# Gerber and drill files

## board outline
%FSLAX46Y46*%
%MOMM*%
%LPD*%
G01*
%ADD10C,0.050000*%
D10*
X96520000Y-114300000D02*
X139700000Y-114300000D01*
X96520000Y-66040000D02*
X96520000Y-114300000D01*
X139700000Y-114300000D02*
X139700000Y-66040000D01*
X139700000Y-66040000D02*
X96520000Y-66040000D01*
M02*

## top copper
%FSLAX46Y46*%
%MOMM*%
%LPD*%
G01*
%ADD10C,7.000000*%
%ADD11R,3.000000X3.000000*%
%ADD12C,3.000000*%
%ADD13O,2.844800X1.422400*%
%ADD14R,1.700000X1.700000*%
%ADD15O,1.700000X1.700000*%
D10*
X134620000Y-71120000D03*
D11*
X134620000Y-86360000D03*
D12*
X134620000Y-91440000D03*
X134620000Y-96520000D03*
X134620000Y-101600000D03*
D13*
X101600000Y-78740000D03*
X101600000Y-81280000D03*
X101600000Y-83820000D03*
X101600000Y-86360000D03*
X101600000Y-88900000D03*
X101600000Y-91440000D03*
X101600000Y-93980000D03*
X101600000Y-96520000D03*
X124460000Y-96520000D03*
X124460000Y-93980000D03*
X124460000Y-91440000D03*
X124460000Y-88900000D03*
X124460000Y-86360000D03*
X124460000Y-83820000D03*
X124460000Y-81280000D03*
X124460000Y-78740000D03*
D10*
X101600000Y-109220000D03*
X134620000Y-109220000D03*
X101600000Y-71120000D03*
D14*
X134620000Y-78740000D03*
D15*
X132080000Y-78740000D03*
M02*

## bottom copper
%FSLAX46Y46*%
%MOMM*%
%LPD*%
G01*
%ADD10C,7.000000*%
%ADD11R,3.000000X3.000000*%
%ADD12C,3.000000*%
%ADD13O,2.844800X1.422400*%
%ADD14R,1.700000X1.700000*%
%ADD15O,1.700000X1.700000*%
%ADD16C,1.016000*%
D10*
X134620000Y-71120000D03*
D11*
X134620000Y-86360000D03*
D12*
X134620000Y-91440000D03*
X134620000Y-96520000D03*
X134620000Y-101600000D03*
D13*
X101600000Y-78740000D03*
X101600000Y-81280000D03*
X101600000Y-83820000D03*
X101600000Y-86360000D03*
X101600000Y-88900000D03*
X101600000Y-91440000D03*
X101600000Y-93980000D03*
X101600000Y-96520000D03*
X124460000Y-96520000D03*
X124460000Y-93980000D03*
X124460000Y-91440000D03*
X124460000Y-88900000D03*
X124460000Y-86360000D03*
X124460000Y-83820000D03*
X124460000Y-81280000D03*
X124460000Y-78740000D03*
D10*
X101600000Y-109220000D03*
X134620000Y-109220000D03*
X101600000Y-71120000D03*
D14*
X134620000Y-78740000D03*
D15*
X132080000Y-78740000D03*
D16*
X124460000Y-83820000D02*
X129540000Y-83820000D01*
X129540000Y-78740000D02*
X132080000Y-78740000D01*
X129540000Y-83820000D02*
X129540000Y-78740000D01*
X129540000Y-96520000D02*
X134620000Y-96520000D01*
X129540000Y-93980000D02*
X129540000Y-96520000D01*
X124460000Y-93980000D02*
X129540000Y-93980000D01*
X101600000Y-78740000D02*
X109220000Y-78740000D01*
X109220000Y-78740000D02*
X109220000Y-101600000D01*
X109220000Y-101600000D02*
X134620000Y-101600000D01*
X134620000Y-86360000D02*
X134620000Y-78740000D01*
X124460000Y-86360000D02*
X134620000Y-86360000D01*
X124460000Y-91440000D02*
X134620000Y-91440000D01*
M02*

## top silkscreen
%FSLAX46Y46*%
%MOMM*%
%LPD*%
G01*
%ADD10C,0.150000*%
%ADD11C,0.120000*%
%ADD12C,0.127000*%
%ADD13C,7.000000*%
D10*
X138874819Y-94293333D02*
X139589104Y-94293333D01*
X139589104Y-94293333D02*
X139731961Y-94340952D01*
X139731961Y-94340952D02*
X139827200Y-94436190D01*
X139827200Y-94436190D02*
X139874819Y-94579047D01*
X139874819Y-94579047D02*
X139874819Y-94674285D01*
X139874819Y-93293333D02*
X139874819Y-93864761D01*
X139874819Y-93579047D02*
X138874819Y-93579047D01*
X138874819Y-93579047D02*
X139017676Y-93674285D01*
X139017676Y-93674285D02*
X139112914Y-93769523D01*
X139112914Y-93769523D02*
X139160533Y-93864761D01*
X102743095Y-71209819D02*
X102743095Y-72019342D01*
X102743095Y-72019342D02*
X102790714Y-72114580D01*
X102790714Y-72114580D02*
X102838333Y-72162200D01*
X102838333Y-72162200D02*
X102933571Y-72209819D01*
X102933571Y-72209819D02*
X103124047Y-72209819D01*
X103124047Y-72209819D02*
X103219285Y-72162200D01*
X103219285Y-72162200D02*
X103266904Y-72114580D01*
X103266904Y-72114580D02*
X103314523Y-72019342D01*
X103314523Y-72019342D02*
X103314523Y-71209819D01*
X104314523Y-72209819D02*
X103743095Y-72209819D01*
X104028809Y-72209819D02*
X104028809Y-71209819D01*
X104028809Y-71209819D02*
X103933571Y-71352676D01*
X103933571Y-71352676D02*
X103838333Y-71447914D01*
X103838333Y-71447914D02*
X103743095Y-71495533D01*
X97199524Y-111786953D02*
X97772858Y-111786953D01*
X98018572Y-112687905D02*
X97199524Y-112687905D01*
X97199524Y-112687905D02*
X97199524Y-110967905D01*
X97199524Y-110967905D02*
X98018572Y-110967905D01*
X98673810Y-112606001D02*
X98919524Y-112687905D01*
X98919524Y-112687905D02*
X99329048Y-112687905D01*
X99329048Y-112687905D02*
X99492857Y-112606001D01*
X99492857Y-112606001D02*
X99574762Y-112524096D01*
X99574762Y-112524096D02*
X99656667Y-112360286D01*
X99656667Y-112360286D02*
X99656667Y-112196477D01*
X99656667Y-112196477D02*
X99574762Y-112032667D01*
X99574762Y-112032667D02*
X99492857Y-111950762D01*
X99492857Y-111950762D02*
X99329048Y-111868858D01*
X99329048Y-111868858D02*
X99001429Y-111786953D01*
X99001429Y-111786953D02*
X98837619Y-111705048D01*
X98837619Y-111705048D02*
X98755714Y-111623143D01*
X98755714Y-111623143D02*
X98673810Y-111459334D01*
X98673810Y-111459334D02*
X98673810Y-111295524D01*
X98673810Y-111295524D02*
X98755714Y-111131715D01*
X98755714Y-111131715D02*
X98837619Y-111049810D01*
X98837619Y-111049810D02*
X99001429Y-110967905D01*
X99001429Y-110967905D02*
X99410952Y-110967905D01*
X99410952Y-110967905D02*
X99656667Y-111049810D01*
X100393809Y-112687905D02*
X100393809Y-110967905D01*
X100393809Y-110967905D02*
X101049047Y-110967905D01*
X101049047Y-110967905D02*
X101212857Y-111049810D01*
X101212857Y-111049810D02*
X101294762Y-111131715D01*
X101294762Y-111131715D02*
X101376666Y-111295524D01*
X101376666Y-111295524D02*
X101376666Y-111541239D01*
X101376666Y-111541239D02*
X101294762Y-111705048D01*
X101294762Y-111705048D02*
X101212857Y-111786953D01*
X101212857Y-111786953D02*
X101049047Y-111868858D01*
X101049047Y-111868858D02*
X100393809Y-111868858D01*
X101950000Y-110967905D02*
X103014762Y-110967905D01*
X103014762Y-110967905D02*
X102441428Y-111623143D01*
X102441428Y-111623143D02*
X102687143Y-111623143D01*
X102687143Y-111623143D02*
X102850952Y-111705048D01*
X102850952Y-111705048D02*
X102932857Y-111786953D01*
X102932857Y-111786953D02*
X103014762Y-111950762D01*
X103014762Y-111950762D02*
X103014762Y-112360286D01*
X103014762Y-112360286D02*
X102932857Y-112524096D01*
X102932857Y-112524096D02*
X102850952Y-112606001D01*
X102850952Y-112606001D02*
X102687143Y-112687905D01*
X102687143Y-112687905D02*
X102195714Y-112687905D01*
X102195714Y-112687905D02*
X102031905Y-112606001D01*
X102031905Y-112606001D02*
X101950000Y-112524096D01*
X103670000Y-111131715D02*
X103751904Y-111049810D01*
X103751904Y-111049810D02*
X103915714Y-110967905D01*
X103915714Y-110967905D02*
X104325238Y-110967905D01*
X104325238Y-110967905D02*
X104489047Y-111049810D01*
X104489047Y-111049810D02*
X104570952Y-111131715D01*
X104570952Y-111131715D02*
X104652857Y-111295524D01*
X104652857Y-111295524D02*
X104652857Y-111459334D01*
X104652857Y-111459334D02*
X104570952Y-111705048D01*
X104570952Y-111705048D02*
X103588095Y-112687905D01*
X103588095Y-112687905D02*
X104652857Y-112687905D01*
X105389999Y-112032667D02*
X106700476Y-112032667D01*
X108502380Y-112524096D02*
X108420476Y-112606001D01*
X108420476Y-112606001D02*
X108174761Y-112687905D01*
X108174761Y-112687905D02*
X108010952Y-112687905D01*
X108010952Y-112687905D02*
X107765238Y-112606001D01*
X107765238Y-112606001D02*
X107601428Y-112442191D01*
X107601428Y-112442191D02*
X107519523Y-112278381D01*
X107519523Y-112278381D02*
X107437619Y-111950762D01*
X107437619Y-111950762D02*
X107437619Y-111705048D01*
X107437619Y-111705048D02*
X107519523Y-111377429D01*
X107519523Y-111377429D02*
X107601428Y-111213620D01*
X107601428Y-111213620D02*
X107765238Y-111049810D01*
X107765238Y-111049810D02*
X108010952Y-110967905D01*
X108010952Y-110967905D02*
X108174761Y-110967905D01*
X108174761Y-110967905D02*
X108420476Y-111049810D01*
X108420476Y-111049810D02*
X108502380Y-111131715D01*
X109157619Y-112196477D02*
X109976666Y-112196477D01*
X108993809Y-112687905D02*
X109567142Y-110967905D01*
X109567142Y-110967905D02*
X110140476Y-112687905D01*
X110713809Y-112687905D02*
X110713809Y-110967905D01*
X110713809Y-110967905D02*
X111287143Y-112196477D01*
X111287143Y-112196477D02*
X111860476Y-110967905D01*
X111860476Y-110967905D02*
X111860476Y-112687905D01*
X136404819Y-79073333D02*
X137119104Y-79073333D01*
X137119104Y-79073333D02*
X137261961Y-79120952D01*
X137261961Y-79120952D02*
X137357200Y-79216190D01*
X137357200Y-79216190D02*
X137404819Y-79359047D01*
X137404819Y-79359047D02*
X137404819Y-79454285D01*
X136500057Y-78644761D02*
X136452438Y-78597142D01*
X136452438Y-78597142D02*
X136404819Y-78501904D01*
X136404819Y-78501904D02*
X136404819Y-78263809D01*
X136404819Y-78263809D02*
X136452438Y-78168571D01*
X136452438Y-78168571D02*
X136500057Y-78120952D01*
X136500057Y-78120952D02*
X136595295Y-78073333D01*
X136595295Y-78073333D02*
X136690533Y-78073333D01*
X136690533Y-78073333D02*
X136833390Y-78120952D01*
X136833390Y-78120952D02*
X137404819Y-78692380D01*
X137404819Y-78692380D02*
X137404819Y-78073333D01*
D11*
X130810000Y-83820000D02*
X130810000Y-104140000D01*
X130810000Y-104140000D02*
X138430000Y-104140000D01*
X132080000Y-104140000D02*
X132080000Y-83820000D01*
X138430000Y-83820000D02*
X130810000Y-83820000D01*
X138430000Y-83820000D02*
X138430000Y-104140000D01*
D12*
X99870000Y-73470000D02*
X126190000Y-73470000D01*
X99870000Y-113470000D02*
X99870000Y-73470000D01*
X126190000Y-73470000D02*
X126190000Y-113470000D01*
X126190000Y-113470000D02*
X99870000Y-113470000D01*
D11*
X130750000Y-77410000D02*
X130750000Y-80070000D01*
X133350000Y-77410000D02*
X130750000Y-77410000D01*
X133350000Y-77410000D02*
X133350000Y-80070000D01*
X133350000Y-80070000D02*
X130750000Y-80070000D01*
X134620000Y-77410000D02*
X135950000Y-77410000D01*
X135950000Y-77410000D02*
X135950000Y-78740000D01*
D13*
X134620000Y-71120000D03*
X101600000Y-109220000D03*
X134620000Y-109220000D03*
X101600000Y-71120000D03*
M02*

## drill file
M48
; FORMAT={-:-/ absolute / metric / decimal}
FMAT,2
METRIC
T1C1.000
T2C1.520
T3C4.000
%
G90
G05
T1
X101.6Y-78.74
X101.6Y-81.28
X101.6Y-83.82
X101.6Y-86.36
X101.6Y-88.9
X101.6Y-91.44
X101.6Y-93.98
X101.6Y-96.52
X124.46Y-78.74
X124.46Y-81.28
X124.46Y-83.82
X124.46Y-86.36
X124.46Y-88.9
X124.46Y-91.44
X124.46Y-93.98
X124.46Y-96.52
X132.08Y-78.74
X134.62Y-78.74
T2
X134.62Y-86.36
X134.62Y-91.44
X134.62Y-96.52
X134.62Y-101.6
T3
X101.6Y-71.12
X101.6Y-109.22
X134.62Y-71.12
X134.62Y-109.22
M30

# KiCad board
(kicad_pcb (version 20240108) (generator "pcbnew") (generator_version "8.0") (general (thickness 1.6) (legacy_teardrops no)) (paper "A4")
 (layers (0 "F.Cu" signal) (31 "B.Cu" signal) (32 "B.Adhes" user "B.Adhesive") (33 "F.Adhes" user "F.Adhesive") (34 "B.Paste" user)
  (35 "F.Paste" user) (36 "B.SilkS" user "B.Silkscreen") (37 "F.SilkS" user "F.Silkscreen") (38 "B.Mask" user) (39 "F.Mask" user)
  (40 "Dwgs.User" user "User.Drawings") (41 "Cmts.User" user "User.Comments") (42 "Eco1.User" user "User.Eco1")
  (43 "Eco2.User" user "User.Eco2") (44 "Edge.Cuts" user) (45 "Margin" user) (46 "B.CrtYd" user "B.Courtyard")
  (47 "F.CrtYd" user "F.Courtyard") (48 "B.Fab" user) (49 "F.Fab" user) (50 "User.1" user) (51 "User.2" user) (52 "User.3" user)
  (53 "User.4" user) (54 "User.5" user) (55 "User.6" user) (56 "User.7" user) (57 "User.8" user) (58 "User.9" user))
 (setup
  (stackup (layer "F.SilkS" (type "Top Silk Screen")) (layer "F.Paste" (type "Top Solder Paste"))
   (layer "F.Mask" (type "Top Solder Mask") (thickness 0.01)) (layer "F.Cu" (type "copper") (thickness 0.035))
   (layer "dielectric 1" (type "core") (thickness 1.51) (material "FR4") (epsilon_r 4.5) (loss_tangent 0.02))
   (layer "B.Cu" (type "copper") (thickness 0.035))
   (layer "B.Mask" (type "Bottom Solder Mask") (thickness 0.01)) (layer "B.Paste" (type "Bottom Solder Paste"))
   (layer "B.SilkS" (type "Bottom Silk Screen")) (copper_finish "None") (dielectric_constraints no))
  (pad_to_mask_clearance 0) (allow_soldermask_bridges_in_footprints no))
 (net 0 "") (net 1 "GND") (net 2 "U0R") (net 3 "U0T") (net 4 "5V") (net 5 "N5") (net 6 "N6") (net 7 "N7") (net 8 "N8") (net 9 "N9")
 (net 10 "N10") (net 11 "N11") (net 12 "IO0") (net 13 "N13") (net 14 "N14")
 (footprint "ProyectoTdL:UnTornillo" (layer "F.Cu") (at 134.62 71.12)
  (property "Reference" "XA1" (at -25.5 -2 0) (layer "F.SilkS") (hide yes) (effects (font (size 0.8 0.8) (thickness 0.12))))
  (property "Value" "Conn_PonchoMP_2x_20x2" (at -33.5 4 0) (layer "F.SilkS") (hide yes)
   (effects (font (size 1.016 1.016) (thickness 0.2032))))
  (pad "~" thru_hole circle (at 0 0) (size 7 7) (drill 4) (layers "*.Cu" "*.Mask" "F.SilkS") (remove_unused_layers no)))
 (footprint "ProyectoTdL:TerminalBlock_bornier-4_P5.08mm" (layer "F.Cu") (at 134.62 86.36 -90)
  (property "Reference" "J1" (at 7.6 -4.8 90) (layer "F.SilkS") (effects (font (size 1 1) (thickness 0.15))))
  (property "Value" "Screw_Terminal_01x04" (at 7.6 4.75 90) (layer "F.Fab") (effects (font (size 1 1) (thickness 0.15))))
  (fp_line (start -2.54 3.81) (end 17.78 3.81) (stroke (width 0.12) (type solid)) (layer "F.SilkS"))
  (fp_line (start 17.78 3.81) (end 17.78 -3.81) (stroke (width 0.12) (type solid)) (layer "F.SilkS"))
  (fp_line (start 17.78 2.54) (end -2.54 2.54) (stroke (width 0.12) (type solid)) (layer "F.SilkS"))
  (fp_line (start -2.54 -3.81) (end -2.54 3.81) (stroke (width 0.12) (type solid)) (layer "F.SilkS"))
  (fp_line (start -2.54 -3.81) (end 17.78 -3.81) (stroke (width 0.12) (type solid)) (layer "F.SilkS"))
  (pad "1" thru_hole rect (at 0 0 270) (size 3 3) (drill 1.52) (layers "*.Cu" "*.Mask") (remove_unused_layers no) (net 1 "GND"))
  (pad "2" thru_hole circle (at 5.08 0 270) (size 3 3) (drill 1.52) (layers "*.Cu" "*.Mask") (remove_unused_layers no) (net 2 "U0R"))
  (pad "3" thru_hole circle (at 10.16 0 270) (size 3 3) (drill 1.52) (layers "*.Cu" "*.Mask") (remove_unused_layers no) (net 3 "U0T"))
  (pad "4" thru_hole circle (at 15.24 0 270) (size 3 3) (drill 1.52) (layers "*.Cu" "*.Mask") (remove_unused_layers no) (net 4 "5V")))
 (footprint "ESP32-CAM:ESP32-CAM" (layer "F.Cu") (at 113.03 88.9)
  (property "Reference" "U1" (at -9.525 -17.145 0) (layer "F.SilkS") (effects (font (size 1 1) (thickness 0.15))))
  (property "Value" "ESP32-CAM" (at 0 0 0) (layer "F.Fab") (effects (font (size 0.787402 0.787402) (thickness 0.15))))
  (fp_line (start -13.16 -15.43) (end 13.16 -15.43) (stroke (width 0.127) (type solid)) (layer "F.SilkS"))
  (fp_line (start -13.16 24.57) (end -13.16 -15.43) (stroke (width 0.127) (type solid)) (layer "F.SilkS"))
  (fp_line (start 13.16 -15.43) (end 13.16 24.57) (stroke (width 0.127) (type solid)) (layer "F.SilkS"))
  (fp_line (start 13.16 24.57) (end -13.16 24.57) (stroke (width 0.127) (type solid)) (layer "F.SilkS"))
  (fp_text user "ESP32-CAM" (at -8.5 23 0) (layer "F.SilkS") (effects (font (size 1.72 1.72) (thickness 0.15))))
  (pad "P$1" thru_hole oval (at -11.43 -10.16) (size 2.8448 1.4224) (drill 1) (layers "*.Cu" "*.Mask") (remove_unused_layers no)
   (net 4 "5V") (solder_mask_margin 0.102))
  (pad "P$2" thru_hole oval (at -11.43 -7.62) (size 2.8448 1.4224) (drill 1) (layers "*.Cu" "*.Mask") (remove_unused_layers no)
   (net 1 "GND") (solder_mask_margin 0.102))
  (pad "P$3" thru_hole oval (at -11.43 -5.08) (size 2.8448 1.4224) (drill 1) (layers "*.Cu" "*.Mask") (remove_unused_layers no) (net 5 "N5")
   (solder_mask_margin 0.102))
  (pad "P$4" thru_hole oval (at -11.43 -2.54) (size 2.8448 1.4224) (drill 1) (layers "*.Cu" "*.Mask") (remove_unused_layers no) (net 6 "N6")
   (solder_mask_margin 0.102))
  (pad "P$5" thru_hole oval (at -11.43 0) (size 2.8448 1.4224) (drill 1) (layers "*.Cu" "*.Mask") (remove_unused_layers no) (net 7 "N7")
   (solder_mask_margin 0.102))
  (pad "P$6" thru_hole oval (at -11.43 2.54) (size 2.8448 1.4224) (drill 1) (layers "*.Cu" "*.Mask") (remove_unused_layers no) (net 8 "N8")
   (solder_mask_margin 0.102))
  (pad "P$7" thru_hole oval (at -11.43 5.08) (size 2.8448 1.4224) (drill 1) (layers "*.Cu" "*.Mask") (remove_unused_layers no) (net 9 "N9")
   (solder_mask_margin 0.102))
  (pad "P$8" thru_hole oval (at -11.43 7.62) (size 2.8448 1.4224) (drill 1) (layers "*.Cu" "*.Mask") (remove_unused_layers no)
   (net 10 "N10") (solder_mask_margin 0.102))
  (pad "P$9" thru_hole oval (at 11.43 7.62) (size 2.8448 1.4224) (drill 1) (layers "*.Cu" "*.Mask") (remove_unused_layers no) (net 1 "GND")
   (solder_mask_margin 0.102))
  (pad "P$10" thru_hole oval (at 11.43 5.08) (size 2.8448 1.4224) (drill 1) (layers "*.Cu" "*.Mask") (remove_unused_layers no) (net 3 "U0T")
   (solder_mask_margin 0.102))
  (pad "P$11" thru_hole oval (at 11.43 2.54) (size 2.8448 1.4224) (drill 1) (layers "*.Cu" "*.Mask") (remove_unused_layers no) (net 2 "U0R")
   (solder_mask_margin 0.102))
  (pad "P$12" thru_hole oval (at 11.43 0) (size 2.8448 1.4224) (drill 1) (layers "*.Cu" "*.Mask") (remove_unused_layers no) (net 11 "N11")
   (solder_mask_margin 0.102))
  (pad "P$13" thru_hole oval (at 11.43 -2.54) (size 2.8448 1.4224) (drill 1) (layers "*.Cu" "*.Mask") (remove_unused_layers no)
   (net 1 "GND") (solder_mask_margin 0.102))
  (pad "P$14" thru_hole oval (at 11.43 -5.08) (size 2.8448 1.4224) (drill 1) (layers "*.Cu" "*.Mask") (remove_unused_layers no)
   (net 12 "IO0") (solder_mask_margin 0.102))
  (pad "P$15" thru_hole oval (at 11.43 -7.62) (size 2.8448 1.4224) (drill 1) (layers "*.Cu" "*.Mask") (remove_unused_layers no)
   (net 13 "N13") (solder_mask_margin 0.102))
  (pad "P$16" thru_hole oval (at 11.43 -10.16) (size 2.8448 1.4224) (drill 1) (layers "*.Cu" "*.Mask") (remove_unused_layers no)
   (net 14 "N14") (solder_mask_margin 0.102)))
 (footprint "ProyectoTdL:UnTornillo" (layer "F.Cu") (at 101.6 109.22)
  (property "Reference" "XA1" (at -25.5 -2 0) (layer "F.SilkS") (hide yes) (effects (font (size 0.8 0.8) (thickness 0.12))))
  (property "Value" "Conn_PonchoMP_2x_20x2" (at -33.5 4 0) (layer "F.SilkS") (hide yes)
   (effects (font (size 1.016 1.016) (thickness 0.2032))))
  (pad "~" thru_hole circle (at 0 0) (size 7 7) (drill 4) (layers "*.Cu" "*.Mask" "F.SilkS") (remove_unused_layers no)))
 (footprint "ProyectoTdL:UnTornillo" (layer "F.Cu") (at 134.62 109.22)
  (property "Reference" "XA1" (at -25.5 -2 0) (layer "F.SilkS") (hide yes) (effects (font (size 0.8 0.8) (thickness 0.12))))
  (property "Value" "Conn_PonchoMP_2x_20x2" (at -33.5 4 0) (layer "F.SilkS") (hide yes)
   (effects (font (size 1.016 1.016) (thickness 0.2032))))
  (pad "~" thru_hole circle (at 0 0) (size 7 7) (drill 4) (layers "*.Cu" "*.Mask" "F.SilkS") (remove_unused_layers no)))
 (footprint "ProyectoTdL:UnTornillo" (layer "F.Cu") (at 101.6 71.12)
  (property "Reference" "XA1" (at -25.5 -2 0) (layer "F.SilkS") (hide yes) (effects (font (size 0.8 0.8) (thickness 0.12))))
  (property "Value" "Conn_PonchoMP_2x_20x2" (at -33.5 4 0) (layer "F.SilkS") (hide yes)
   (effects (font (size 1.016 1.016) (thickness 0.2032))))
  (pad "~" thru_hole circle (at 0 0) (size 7 7) (drill 4) (layers "*.Cu" "*.Mask" "F.SilkS") (remove_unused_layers no)))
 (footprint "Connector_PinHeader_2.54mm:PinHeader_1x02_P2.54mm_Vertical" (layer "F.Cu") (at 134.62 78.74 -90)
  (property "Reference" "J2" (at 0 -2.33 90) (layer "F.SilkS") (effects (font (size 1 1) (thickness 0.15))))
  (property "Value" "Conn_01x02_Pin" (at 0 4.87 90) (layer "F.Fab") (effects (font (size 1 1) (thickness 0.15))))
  (fp_line (start -1.33 3.87) (end 1.33 3.87) (stroke (width 0.12) (type solid)) (layer "F.SilkS"))
  (fp_line (start -1.33 1.27) (end -1.33 3.87) (stroke (width 0.12) (type solid)) (layer "F.SilkS"))
  (fp_line (start -1.33 1.27) (end 1.33 1.27) (stroke (width 0.12) (type solid)) (layer "F.SilkS"))
  (fp_line (start 1.33 1.27) (end 1.33 3.87) (stroke (width 0.12) (type solid)) (layer "F.SilkS"))
  (fp_line (start -1.33 0) (end -1.33 -1.33) (stroke (width 0.12) (type solid)) (layer "F.SilkS"))
  (fp_line (start -1.33 -1.33) (end 0 -1.33) (stroke (width 0.12) (type solid)) (layer "F.SilkS"))
  (pad "1" thru_hole rect (at 0 0 270) (size 1.7 1.7) (drill 1) (layers "*.Cu" "*.Mask") (remove_unused_layers no) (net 1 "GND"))
  (pad "2" thru_hole oval (at 0 2.54 270) (size 1.7 1.7) (drill 1) (layers "*.Cu" "*.Mask") (remove_unused_layers no) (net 12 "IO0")))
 (gr_line (start 96.52 114.3) (end 139.7 114.3) (stroke (width 0.05) (type default)) (layer "Edge.Cuts"))
 (gr_line (start 96.52 66.04) (end 96.52 114.3) (stroke (width 0.05) (type default)) (layer "Edge.Cuts"))
 (gr_line (start 139.7 114.3) (end 139.7 66.04) (stroke (width 0.05) (type default)) (layer "Edge.Cuts"))
 (gr_line (start 139.7 66.04) (end 96.52 66.04) (stroke (width 0.05) (type default)) (layer "Edge.Cuts"))
 (segment (start 124.46 83.82) (end 129.54 83.82) (width 1.016) (layer "B.Cu") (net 12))
 (segment (start 129.54 78.74) (end 132.08 78.74) (width 1.016) (layer "B.Cu") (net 12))
 (segment (start 129.54 83.82) (end 129.54 78.74) (width 1.016) (layer "B.Cu") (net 12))
 (segment (start 129.54 96.52) (end 134.62 96.52) (width 1.016) (layer "B.Cu") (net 3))
 (segment (start 129.54 93.98) (end 129.54 96.52) (width 1.016) (layer "B.Cu") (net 3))
 (segment (start 124.46 93.98) (end 129.54 93.98) (width 1.016) (layer "B.Cu") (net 3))
 (segment (start 101.6 78.74) (end 109.22 78.74) (width 1.016) (layer "B.Cu") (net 4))
 (segment (start 109.22 78.74) (end 109.22 101.6) (width 1.016) (layer "B.Cu") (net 4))
 (segment (start 109.22 101.6) (end 134.62 101.6) (width 1.016) (layer "B.Cu") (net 4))
 (segment (start 134.62 86.36) (end 134.62 78.74) (width 1.016) (layer "B.Cu") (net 1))
 (segment (start 124.46 86.36) (end 134.62 86.36) (width 1.016) (layer "B.Cu") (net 1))
 (segment (start 124.46 91.44) (end 134.62 91.44) (width 1.016) (layer "B.Cu") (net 2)))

